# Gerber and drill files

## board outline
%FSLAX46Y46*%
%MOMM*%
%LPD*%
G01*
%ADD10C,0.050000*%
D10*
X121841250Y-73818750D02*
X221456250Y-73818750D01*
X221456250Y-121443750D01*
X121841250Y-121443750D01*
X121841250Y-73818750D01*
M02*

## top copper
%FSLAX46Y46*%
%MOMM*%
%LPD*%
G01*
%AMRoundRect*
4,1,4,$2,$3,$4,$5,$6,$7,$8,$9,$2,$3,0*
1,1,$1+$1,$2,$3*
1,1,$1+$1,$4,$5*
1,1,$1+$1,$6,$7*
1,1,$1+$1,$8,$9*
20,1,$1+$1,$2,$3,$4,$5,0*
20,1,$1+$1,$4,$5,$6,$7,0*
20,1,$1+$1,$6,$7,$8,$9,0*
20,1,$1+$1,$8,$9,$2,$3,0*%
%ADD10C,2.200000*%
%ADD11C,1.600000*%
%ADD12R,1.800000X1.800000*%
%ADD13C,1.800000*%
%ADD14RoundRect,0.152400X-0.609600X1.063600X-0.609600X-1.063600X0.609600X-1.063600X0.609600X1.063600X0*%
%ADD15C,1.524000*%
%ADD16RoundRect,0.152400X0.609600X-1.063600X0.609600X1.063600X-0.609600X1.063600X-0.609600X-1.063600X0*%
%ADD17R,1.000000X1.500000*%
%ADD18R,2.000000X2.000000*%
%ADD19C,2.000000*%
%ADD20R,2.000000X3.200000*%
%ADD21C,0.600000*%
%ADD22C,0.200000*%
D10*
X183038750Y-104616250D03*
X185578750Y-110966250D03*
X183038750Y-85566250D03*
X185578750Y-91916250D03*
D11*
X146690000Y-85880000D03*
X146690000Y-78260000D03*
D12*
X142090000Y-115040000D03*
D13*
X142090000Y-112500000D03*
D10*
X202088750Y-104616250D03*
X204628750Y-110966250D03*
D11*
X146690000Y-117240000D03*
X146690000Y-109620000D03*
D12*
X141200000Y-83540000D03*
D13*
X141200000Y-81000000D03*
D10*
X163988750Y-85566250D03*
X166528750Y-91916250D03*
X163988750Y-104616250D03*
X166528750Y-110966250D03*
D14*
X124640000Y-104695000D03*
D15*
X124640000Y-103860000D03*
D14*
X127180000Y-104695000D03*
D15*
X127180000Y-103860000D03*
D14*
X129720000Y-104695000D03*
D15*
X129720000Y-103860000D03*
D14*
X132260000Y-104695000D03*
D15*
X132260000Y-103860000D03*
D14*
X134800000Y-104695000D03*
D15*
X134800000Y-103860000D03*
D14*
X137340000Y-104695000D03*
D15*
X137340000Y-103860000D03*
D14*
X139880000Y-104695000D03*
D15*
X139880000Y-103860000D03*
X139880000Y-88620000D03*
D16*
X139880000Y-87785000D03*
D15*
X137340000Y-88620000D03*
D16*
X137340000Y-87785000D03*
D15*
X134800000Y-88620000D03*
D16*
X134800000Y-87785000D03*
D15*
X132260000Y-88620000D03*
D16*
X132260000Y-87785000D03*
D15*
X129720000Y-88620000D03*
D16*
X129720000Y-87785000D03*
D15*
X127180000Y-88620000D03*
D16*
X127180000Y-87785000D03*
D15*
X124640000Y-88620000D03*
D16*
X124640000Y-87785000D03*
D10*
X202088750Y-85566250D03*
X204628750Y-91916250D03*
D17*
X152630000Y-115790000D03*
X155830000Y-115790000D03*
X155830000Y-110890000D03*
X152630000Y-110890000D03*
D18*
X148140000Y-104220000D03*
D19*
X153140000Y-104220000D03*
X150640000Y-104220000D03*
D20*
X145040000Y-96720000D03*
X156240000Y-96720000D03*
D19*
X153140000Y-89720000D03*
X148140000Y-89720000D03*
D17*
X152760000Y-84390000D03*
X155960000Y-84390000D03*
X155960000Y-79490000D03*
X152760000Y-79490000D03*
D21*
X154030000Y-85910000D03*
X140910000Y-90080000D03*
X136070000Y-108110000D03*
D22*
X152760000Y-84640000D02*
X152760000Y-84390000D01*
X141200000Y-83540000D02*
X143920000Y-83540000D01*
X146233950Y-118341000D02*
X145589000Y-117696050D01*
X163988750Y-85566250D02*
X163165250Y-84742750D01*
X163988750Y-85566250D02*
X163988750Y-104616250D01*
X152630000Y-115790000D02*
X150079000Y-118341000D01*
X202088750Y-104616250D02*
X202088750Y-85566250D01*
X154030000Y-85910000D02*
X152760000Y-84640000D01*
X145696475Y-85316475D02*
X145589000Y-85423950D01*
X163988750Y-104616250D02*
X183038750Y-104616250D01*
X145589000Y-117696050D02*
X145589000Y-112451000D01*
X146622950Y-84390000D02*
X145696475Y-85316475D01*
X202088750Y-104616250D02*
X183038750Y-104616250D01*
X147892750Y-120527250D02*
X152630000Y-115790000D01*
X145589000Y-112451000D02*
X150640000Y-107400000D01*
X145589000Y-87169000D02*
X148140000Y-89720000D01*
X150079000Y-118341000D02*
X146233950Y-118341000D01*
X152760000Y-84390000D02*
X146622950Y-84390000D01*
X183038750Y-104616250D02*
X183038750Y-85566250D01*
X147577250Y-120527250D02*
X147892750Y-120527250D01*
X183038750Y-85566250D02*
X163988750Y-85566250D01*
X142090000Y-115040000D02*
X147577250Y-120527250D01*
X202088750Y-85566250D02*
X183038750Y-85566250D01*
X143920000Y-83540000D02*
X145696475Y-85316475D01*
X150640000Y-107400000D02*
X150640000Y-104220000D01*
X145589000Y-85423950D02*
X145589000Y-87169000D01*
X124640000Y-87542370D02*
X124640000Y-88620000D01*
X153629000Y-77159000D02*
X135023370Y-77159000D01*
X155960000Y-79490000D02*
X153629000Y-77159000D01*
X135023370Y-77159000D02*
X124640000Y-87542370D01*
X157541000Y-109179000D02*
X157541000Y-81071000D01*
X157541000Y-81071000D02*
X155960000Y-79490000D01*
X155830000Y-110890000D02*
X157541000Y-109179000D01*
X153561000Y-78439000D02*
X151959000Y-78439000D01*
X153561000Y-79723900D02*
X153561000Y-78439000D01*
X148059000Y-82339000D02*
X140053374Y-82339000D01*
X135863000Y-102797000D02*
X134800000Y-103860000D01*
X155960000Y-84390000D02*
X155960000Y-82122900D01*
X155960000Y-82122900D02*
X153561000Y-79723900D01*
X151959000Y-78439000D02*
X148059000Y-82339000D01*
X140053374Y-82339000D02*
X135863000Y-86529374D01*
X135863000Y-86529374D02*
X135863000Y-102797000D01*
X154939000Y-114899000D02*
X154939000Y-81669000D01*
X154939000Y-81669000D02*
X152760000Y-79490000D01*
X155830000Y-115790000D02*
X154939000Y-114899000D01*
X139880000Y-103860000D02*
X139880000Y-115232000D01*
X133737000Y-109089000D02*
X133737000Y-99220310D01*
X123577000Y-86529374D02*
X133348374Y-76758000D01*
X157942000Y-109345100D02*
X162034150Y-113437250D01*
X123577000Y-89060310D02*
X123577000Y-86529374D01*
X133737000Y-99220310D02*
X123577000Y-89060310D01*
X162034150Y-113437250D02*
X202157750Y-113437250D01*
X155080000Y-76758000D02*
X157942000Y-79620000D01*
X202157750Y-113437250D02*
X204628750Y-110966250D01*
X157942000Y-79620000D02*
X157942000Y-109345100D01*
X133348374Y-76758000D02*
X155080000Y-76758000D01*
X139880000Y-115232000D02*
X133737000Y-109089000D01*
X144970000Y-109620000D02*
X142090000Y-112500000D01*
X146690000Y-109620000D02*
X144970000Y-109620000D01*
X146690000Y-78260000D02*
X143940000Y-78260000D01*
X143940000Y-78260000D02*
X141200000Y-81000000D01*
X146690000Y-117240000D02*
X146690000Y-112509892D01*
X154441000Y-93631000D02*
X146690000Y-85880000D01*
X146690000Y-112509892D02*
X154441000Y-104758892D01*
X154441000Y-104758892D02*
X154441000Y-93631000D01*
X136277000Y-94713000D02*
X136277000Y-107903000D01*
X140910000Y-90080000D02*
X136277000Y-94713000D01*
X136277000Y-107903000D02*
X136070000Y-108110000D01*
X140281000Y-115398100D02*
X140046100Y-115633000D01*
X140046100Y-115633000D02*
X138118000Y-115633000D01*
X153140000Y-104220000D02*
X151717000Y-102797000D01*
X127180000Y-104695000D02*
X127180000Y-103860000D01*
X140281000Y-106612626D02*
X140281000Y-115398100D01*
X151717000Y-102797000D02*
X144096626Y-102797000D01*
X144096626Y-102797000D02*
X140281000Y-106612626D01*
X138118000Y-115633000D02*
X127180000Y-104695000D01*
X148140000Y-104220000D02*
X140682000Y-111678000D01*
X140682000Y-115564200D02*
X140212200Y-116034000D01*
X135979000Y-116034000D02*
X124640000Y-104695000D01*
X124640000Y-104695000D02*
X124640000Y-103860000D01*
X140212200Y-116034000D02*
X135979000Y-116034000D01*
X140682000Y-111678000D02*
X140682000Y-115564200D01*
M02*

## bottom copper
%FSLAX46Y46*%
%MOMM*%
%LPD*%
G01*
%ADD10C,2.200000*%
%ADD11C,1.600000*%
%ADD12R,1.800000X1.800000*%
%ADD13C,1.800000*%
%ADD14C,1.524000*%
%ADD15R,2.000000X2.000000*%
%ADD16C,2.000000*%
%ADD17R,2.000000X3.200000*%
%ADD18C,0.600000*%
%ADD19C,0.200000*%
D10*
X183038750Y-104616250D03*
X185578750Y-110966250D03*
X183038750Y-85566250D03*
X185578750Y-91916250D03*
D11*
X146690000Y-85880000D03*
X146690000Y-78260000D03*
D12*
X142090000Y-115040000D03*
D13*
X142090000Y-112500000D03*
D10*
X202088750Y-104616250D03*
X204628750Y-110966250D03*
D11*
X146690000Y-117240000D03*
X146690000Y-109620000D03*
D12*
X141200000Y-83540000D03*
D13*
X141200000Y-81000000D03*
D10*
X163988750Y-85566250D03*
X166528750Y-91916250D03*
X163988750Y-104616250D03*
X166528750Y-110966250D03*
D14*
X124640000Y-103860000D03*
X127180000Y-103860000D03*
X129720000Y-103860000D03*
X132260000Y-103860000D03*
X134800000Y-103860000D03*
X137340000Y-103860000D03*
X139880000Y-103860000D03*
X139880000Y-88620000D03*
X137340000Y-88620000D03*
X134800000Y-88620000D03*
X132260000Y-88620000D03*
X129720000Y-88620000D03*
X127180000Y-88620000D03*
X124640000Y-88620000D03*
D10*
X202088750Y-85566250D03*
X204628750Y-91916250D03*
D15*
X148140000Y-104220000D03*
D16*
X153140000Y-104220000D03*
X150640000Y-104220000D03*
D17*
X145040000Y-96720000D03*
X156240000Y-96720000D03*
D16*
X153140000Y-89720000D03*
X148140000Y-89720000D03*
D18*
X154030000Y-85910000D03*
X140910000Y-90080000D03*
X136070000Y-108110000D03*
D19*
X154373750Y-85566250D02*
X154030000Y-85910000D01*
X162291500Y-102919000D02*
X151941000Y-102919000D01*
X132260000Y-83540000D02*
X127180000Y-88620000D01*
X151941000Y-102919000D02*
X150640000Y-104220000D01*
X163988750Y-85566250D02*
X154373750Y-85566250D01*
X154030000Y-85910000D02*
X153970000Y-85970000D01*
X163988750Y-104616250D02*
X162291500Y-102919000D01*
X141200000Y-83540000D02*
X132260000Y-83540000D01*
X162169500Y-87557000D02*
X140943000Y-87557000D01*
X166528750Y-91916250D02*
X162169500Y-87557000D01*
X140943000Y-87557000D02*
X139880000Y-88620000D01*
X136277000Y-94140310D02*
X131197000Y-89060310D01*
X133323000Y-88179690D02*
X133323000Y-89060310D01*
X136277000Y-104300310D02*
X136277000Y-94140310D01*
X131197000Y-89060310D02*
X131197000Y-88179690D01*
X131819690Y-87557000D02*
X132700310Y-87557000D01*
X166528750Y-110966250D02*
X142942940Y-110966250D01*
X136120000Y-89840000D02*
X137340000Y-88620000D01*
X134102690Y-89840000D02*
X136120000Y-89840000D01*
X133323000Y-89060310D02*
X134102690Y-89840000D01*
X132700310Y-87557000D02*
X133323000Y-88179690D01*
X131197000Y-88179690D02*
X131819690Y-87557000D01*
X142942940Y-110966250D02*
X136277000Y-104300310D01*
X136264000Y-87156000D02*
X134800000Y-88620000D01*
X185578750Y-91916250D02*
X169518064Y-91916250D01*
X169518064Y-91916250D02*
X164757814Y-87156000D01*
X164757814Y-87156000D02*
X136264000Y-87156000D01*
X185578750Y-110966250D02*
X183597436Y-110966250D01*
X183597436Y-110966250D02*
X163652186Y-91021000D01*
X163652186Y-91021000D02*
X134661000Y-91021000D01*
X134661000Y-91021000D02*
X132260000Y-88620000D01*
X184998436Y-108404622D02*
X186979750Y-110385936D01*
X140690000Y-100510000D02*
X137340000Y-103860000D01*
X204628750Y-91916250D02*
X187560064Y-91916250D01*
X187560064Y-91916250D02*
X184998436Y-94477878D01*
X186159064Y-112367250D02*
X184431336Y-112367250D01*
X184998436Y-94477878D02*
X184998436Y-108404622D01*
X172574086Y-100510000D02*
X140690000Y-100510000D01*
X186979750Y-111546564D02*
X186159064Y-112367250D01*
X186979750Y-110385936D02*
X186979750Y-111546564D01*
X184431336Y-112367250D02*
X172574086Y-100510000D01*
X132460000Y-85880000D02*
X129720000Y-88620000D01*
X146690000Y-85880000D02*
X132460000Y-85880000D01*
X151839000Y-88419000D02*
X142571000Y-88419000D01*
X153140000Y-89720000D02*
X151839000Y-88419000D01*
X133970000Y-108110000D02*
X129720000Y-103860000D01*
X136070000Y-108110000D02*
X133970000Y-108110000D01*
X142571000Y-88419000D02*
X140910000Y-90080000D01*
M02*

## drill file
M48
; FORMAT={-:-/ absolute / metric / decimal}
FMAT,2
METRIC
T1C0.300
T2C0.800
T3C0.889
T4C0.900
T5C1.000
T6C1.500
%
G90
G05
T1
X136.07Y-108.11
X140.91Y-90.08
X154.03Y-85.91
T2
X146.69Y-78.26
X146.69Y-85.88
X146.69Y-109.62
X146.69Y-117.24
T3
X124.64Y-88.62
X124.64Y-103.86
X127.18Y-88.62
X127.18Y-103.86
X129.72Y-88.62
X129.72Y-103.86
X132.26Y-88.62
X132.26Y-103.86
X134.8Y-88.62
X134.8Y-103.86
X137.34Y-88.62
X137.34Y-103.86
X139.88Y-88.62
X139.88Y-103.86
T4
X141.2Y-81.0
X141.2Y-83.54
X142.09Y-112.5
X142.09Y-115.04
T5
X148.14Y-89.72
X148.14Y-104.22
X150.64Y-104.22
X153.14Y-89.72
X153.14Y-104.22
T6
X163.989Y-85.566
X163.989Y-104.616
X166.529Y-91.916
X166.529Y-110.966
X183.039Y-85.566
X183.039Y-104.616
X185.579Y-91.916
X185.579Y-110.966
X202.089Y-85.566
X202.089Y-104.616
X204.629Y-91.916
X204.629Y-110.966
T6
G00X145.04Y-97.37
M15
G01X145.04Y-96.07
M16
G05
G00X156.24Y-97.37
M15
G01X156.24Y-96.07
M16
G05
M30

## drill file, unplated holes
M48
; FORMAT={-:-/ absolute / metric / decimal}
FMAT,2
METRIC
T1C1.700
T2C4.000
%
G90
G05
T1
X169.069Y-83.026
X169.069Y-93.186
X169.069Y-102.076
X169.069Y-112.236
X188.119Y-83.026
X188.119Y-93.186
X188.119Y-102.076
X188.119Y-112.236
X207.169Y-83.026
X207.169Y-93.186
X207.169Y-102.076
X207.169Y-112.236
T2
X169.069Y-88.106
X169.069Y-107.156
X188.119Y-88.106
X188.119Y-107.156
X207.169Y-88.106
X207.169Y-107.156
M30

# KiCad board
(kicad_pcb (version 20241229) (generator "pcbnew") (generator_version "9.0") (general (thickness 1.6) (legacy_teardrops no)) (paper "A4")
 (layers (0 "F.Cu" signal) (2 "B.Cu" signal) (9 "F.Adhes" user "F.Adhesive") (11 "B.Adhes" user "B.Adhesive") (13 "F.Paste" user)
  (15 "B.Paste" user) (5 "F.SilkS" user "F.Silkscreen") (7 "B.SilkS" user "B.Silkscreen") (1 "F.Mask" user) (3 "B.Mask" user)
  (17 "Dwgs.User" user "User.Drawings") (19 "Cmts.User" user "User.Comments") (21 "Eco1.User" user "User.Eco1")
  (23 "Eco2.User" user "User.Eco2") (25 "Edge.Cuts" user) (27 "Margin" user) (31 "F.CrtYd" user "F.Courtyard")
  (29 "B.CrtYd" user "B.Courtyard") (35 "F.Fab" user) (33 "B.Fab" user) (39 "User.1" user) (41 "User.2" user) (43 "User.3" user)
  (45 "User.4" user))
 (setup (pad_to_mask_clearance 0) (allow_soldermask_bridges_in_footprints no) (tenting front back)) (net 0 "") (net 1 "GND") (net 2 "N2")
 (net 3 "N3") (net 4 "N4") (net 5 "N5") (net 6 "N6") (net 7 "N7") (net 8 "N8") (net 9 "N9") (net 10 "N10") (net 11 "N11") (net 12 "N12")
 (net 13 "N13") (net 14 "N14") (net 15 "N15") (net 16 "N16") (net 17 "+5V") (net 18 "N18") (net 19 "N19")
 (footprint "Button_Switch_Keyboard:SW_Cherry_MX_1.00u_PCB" (layer "F.Cu") (at 183.03875 104.61625 90)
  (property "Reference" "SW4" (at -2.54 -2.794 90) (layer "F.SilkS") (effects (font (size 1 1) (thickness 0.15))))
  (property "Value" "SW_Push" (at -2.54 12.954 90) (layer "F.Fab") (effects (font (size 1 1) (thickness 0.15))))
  (pad "" np_thru_hole circle (at -7.62 5.08 90) (size 1.7 1.7) (drill 1.7) (layers "*.Cu" "*.Mask"))
  (pad "" np_thru_hole circle (at -2.54 5.08 90) (size 4 4) (drill 4) (layers "*.Cu" "*.Mask"))
  (pad "" np_thru_hole circle (at 2.54 5.08 90) (size 1.7 1.7) (drill 1.7) (layers "*.Cu" "*.Mask"))
  (pad "1" thru_hole circle (at 0 0 90) (size 2.2 2.2) (drill 1.5) (layers "*.Cu" "*.Mask") (remove_unused_layers no) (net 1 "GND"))
  (pad "2" thru_hole circle (at -6.35 2.54 90) (size 2.2 2.2) (drill 1.5) (layers "*.Cu" "*.Mask") (remove_unused_layers no) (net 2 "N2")))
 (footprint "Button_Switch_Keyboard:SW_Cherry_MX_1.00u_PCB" (layer "F.Cu") (at 183.03875 85.56625 90)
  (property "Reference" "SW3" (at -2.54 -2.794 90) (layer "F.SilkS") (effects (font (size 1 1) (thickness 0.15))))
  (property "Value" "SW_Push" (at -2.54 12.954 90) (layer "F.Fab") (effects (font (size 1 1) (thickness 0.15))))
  (pad "" np_thru_hole circle (at -7.62 5.08 90) (size 1.7 1.7) (drill 1.7) (layers "*.Cu" "*.Mask"))
  (pad "" np_thru_hole circle (at -2.54 5.08 90) (size 4 4) (drill 4) (layers "*.Cu" "*.Mask"))
  (pad "" np_thru_hole circle (at 2.54 5.08 90) (size 1.7 1.7) (drill 1.7) (layers "*.Cu" "*.Mask"))
  (pad "1" thru_hole circle (at 0 0 90) (size 2.2 2.2) (drill 1.5) (layers "*.Cu" "*.Mask") (remove_unused_layers no) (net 1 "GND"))
  (pad "2" thru_hole circle (at -6.35 2.54 90) (size 2.2 2.2) (drill 1.5) (layers "*.Cu" "*.Mask") (remove_unused_layers no) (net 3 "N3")))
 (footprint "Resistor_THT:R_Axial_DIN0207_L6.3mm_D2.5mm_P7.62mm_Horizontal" (layer "F.Cu") (at 146.69 85.88 90)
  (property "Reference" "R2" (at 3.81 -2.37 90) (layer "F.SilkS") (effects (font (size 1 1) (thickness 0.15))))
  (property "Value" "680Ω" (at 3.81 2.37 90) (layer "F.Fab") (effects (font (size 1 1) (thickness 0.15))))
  (pad "1" thru_hole circle (at 0 0 90) (size 1.6 1.6) (drill 0.8) (layers "*.Cu" "*.Mask") (remove_unused_layers no) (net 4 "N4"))
  (pad "2" thru_hole circle (at 7.62 0 90) (size 1.6 1.6) (drill 0.8) (layers "*.Cu" "*.Mask") (remove_unused_layers no) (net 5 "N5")))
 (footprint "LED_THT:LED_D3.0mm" (layer "F.Cu") (at 142.09 115.04 90)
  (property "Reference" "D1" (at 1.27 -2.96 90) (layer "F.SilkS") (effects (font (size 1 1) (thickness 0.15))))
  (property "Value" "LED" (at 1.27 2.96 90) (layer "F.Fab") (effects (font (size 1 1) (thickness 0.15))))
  (pad "1" thru_hole rect (at 0 0 90) (size 1.8 1.8) (drill 0.9) (layers "*.Cu" "*.Mask") (remove_unused_layers no) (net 1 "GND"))
  (pad "2" thru_hole circle (at 2.54 0 90) (size 1.8 1.8) (drill 0.9) (layers "*.Cu" "*.Mask") (remove_unused_layers no) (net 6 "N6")))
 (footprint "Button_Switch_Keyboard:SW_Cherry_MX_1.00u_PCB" (layer "F.Cu") (at 202.08875 104.61625 90)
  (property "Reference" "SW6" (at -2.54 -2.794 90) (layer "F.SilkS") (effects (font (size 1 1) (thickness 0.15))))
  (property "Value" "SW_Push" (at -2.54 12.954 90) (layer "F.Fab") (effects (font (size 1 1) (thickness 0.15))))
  (pad "" np_thru_hole circle (at -7.62 5.08 90) (size 1.7 1.7) (drill 1.7) (layers "*.Cu" "*.Mask"))
  (pad "" np_thru_hole circle (at -2.54 5.08 90) (size 4 4) (drill 4) (layers "*.Cu" "*.Mask"))
  (pad "" np_thru_hole circle (at 2.54 5.08 90) (size 1.7 1.7) (drill 1.7) (layers "*.Cu" "*.Mask"))
  (pad "1" thru_hole circle (at 0 0 90) (size 2.2 2.2) (drill 1.5) (layers "*.Cu" "*.Mask") (remove_unused_layers no) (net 1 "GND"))
  (pad "2" thru_hole circle (at -6.35 2.54 90) (size 2.2 2.2) (drill 1.5) (layers "*.Cu" "*.Mask") (remove_unused_layers no) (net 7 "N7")))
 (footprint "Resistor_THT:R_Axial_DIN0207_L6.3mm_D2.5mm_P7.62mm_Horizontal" (layer "F.Cu") (at 146.69 117.24 90)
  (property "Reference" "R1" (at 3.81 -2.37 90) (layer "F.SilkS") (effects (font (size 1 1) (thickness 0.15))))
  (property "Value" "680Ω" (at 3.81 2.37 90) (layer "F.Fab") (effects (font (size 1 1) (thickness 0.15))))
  (pad "1" thru_hole circle (at 0 0 90) (size 1.6 1.6) (drill 0.8) (layers "*.Cu" "*.Mask") (remove_unused_layers no) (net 4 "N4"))
  (pad "2" thru_hole circle (at 7.62 0 90) (size 1.6 1.6) (drill 0.8) (layers "*.Cu" "*.Mask") (remove_unused_layers no) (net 6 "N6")))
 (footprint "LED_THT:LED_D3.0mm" (layer "F.Cu") (at 141.2 83.54 90)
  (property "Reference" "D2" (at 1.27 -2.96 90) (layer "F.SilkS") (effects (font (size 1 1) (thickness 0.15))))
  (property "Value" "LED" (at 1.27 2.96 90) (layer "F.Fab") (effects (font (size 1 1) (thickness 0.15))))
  (pad "1" thru_hole rect (at 0 0 90) (size 1.8 1.8) (drill 0.9) (layers "*.Cu" "*.Mask") (remove_unused_layers no) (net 1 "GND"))
  (pad "2" thru_hole circle (at 2.54 0 90) (size 1.8 1.8) (drill 0.9) (layers "*.Cu" "*.Mask") (remove_unused_layers no) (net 5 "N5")))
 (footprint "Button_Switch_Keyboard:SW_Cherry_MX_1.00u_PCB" (layer "F.Cu") (at 163.98875 85.56625 90)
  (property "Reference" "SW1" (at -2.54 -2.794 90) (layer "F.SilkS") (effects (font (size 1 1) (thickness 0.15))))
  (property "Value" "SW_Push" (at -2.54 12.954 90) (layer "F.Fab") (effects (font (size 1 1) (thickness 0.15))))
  (pad "" np_thru_hole circle (at -7.62 5.08 90) (size 1.7 1.7) (drill 1.7) (layers "*.Cu" "*.Mask"))
  (pad "" np_thru_hole circle (at -2.54 5.08 90) (size 4 4) (drill 4) (layers "*.Cu" "*.Mask"))
  (pad "" np_thru_hole circle (at 2.54 5.08 90) (size 1.7 1.7) (drill 1.7) (layers "*.Cu" "*.Mask"))
  (pad "1" thru_hole circle (at 0 0 90) (size 2.2 2.2) (drill 1.5) (layers "*.Cu" "*.Mask") (remove_unused_layers no) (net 1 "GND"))
  (pad "2" thru_hole circle (at -6.35 2.54 90) (size 2.2 2.2) (drill 1.5) (layers "*.Cu" "*.Mask") (remove_unused_layers no) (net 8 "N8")))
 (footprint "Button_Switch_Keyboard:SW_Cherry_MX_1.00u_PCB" (layer "F.Cu") (at 163.98875 104.61625 90)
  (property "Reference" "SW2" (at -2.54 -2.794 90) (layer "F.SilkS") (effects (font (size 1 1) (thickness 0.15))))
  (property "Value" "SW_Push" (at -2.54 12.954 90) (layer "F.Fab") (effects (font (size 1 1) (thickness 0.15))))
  (pad "" np_thru_hole circle (at -7.62 5.08 90) (size 1.7 1.7) (drill 1.7) (layers "*.Cu" "*.Mask"))
  (pad "" np_thru_hole circle (at -2.54 5.08 90) (size 4 4) (drill 4) (layers "*.Cu" "*.Mask"))
  (pad "" np_thru_hole circle (at 2.54 5.08 90) (size 1.7 1.7) (drill 1.7) (layers "*.Cu" "*.Mask"))
  (pad "1" thru_hole circle (at 0 0 90) (size 2.2 2.2) (drill 1.5) (layers "*.Cu" "*.Mask") (remove_unused_layers no) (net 1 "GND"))
  (pad "2" thru_hole circle (at -6.35 2.54 90) (size 2.2 2.2) (drill 1.5) (layers "*.Cu" "*.Mask") (remove_unused_layers no) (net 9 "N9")))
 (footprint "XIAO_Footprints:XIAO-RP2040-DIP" (layer "F.Cu") (at 132.26 96.24 90)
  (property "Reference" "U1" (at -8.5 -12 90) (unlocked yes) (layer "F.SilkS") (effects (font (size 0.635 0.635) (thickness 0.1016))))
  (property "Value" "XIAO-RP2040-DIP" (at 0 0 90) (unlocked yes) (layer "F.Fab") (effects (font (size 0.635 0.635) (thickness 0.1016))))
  (pad "1" smd roundrect (at -8.455 -7.62 270) (size 2.432 1.524) (layers "F.Cu" "F.Mask") (roundrect_rratio 0.1) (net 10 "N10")
   (thermal_bridge_angle 45))
  (pad "1" thru_hole circle (at -7.62 -7.62 270) (size 1.524 1.524) (drill 0.889) (layers "*.Cu" "*.Mask") (remove_unused_layers no)
   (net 10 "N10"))
  (pad "2" smd roundrect (at -8.455 -5.08 270) (size 2.432 1.524) (layers "F.Cu" "F.Mask") (roundrect_rratio 0.1) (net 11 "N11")
   (thermal_bridge_angle 45))
  (pad "2" thru_hole circle (at -7.62 -5.08 270) (size 1.524 1.524) (drill 0.889) (layers "*.Cu" "*.Mask") (remove_unused_layers no)
   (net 11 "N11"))
  (pad "3" smd roundrect (at -8.455 -2.54 270) (size 2.432 1.524) (layers "F.Cu" "F.Mask") (roundrect_rratio 0.1) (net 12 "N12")
   (thermal_bridge_angle 45))
  (pad "3" thru_hole circle (at -7.62 -2.54 270) (size 1.524 1.524) (drill 0.889) (layers "*.Cu" "*.Mask") (remove_unused_layers no)
   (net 12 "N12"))
  (pad "4" smd roundrect (at -8.455 0 270) (size 2.432 1.524) (layers "F.Cu" "F.Mask") (roundrect_rratio 0.1) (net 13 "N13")
   (thermal_bridge_angle 45))
  (pad "4" thru_hole circle (at -7.62 0 270) (size 1.524 1.524) (drill 0.889) (layers "*.Cu" "*.Mask") (remove_unused_layers no)
   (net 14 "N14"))
  (pad "5" smd roundrect (at -8.455 2.54 270) (size 2.432 1.524) (layers "F.Cu" "F.Mask") (roundrect_rratio 0.1) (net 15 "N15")
   (thermal_bridge_angle 45))
  (pad "5" thru_hole circle (at -7.62 2.54 270) (size 1.524 1.524) (drill 0.889) (layers "*.Cu" "*.Mask") (remove_unused_layers no)
   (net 15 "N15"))
  (pad "6" smd roundrect (at -8.455 5.08 270) (size 2.432 1.524) (layers "F.Cu" "F.Mask") (roundrect_rratio 0.1) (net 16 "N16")
   (thermal_bridge_angle 45))
  (pad "6" thru_hole circle (at -7.62 5.08 270) (size 1.524 1.524) (drill 0.889) (layers "*.Cu" "*.Mask") (remove_unused_layers no)
   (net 16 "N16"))
  (pad "7" smd roundrect (at -8.455 7.62 270) (size 2.432 1.524) (layers "F.Cu" "F.Mask") (roundrect_rratio 0.1) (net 7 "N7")
   (thermal_bridge_angle 45))
  (pad "7" thru_hole circle (at -7.62 7.62 270) (size 1.524 1.524) (drill 0.889) (layers "*.Cu" "*.Mask") (remove_unused_layers no)
   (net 7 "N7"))
  (pad "8" thru_hole circle (at 7.62 7.62 90) (size 1.524 1.524) (drill 0.889) (layers "*.Cu" "*.Mask") (remove_unused_layers no)
   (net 8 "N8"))
  (pad "8" smd roundrect (at 8.455 7.62 90) (size 2.432 1.524) (layers "F.Cu" "F.Mask") (roundrect_rratio 0.1) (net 8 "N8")
   (thermal_bridge_angle 45))
  (pad "9" thru_hole circle (at 7.62 5.08 90) (size 1.524 1.524) (drill 0.889) (layers "*.Cu" "*.Mask") (remove_unused_layers no)
   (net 9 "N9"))
  (pad "9" smd roundrect (at 8.455 5.08 90) (size 2.432 1.524) (layers "F.Cu" "F.Mask") (roundrect_rratio 0.1) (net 9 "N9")
   (thermal_bridge_angle 45))
  (pad "10" thru_hole circle (at 7.62 2.54 90) (size 1.524 1.524) (drill 0.889) (layers "*.Cu" "*.Mask") (remove_unused_layers no)
   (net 3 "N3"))
  (pad "10" smd roundrect (at 8.455 2.54 90) (size 2.432 1.524) (layers "F.Cu" "F.Mask") (roundrect_rratio 0.1) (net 3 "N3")
   (thermal_bridge_angle 45))
  (pad "11" thru_hole circle (at 7.62 0 90) (size 1.524 1.524) (drill 0.889) (layers "*.Cu" "*.Mask") (remove_unused_layers no) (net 2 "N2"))
  (pad "11" smd roundrect (at 8.455 0 90) (size 2.432 1.524) (layers "F.Cu" "F.Mask") (roundrect_rratio 0.1) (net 2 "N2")
   (thermal_bridge_angle 45))
  (pad "12" thru_hole circle (at 7.62 -2.54 90) (size 1.524 1.524) (drill 0.889) (layers "*.Cu" "*.Mask") (remove_unused_layers no)
   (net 4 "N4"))
  (pad "12" smd roundrect (at 8.455 -2.54 90) (size 2.432 1.524) (layers "F.Cu" "F.Mask") (roundrect_rratio 0.1) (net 4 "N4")
   (thermal_bridge_angle 45))
  (pad "13" thru_hole circle (at 7.62 -5.08 90) (size 1.524 1.524) (drill 0.889) (layers "*.Cu" "*.Mask") (remove_unused_layers no)
   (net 1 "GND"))
  (pad "13" smd roundrect (at 8.455 -5.08 90) (size 2.432 1.524) (layers "F.Cu" "F.Mask") (roundrect_rratio 0.1) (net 1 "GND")
   (thermal_bridge_angle 45))
  (pad "14" thru_hole circle (at 7.62 -7.62 90) (size 1.524 1.524) (drill 0.889) (layers "*.Cu" "*.Mask") (remove_unused_layers no)
   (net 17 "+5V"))
  (pad "14" smd roundrect (at 8.455 -7.62 90) (size 2.432 1.524) (layers "F.Cu" "F.Mask") (roundrect_rratio 0.1) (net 17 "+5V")
   (thermal_bridge_angle 45)))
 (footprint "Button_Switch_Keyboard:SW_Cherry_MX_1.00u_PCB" (layer "F.Cu") (at 202.08875 85.56625 90)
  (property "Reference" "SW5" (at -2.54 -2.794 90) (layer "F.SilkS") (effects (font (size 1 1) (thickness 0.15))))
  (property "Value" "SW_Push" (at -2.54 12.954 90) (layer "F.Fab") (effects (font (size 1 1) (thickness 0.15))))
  (pad "" np_thru_hole circle (at -7.62 5.08 90) (size 1.7 1.7) (drill 1.7) (layers "*.Cu" "*.Mask"))
  (pad "" np_thru_hole circle (at -2.54 5.08 90) (size 4 4) (drill 4) (layers "*.Cu" "*.Mask"))
  (pad "" np_thru_hole circle (at 2.54 5.08 90) (size 1.7 1.7) (drill 1.7) (layers "*.Cu" "*.Mask"))
  (pad "1" thru_hole circle (at 0 0 90) (size 2.2 2.2) (drill 1.5) (layers "*.Cu" "*.Mask") (remove_unused_layers no) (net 1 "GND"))
  (pad "2" thru_hole circle (at -6.35 2.54 90) (size 2.2 2.2) (drill 1.5) (layers "*.Cu" "*.Mask") (remove_unused_layers no) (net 16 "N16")))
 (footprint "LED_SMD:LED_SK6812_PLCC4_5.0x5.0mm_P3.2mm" (layer "F.Cu") (at 154.23 113.34 90)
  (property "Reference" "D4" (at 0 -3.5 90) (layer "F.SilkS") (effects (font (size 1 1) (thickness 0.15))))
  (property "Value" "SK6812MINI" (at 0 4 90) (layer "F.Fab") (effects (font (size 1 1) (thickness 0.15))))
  (pad "1" smd rect (at -2.45 -1.6 270) (size 1.5 1) (layers "F.Cu" "F.Mask" "F.Paste") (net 1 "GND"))
  (pad "2" smd rect (at -2.45 1.6 270) (size 1.5 1) (layers "F.Cu" "F.Mask" "F.Paste") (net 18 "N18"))
  (pad "3" smd rect (at 2.45 1.6 270) (size 1.5 1) (layers "F.Cu" "F.Mask" "F.Paste") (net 17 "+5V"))
  (pad "4" smd rect (at 2.45 -1.6 270) (size 1.5 1) (layers "F.Cu" "F.Mask" "F.Paste") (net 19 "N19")))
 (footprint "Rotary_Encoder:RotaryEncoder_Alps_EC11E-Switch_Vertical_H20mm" (layer "F.Cu") (at 148.14 104.22 90)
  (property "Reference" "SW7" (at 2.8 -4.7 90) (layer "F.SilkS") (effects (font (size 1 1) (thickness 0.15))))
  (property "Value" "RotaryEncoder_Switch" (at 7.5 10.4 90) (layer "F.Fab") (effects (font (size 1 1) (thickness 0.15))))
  (pad "A" thru_hole rect (at 0 0 90) (size 2 2) (drill 1) (layers "*.Cu" "*.Mask") (remove_unused_layers no) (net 10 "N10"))
  (pad "B" thru_hole circle (at 0 5 90) (size 2 2) (drill 1) (layers "*.Cu" "*.Mask") (remove_unused_layers no) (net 11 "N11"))
  (pad "C" thru_hole circle (at 0 2.5 90) (size 2 2) (drill 1) (layers "*.Cu" "*.Mask") (remove_unused_layers no) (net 1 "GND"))
  (pad "MP" thru_hole rect (at 7.5 -3.1 90) (size 3.2 2) (drill oval 2.8 1.5) (layers "*.Cu" "*.Mask") (remove_unused_layers no))
  (pad "MP" thru_hole rect (at 7.5 8.1 90) (size 3.2 2) (drill oval 2.8 1.5) (layers "*.Cu" "*.Mask") (remove_unused_layers no))
  (pad "S1" thru_hole circle (at 14.5 5 90) (size 2 2) (drill 1) (layers "*.Cu" "*.Mask") (remove_unused_layers no) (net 12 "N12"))
  (pad "S2" thru_hole circle (at 14.5 0 90) (size 2 2) (drill 1) (layers "*.Cu" "*.Mask") (remove_unused_layers no) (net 1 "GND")))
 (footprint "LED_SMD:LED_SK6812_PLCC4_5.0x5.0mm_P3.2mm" (layer "F.Cu") (at 154.36 81.94 90)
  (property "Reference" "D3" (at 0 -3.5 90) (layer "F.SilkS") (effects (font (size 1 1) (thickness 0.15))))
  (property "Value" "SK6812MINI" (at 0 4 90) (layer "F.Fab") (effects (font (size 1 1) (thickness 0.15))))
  (pad "1" smd rect (at -2.45 -1.6 270) (size 1.5 1) (layers "F.Cu" "F.Mask" "F.Paste") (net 1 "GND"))
  (pad "2" smd rect (at -2.45 1.6 270) (size 1.5 1) (layers "F.Cu" "F.Mask" "F.Paste") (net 15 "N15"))
  (pad "3" smd rect (at 2.45 1.6 270) (size 1.5 1) (layers "F.Cu" "F.Mask" "F.Paste") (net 17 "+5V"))
  (pad "4" smd rect (at 2.45 -1.6 270) (size 1.5 1) (layers "F.Cu" "F.Mask" "F.Paste") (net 18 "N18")))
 (gr_rect (start 121.84125 73.81875) (end 221.45625 121.44375) (stroke (width 0.05) (type default)) (fill no) (layer "Edge.Cuts"))
 (segment (start 152.76 84.64) (end 152.76 84.39) (width 0.2) (layer "F.Cu") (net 1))
 (segment (start 141.2 83.54) (end 143.92 83.54) (width 0.2) (layer "F.Cu") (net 1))
 (segment (start 146.23395 118.341) (end 145.589 117.69605) (width 0.2) (layer "F.Cu") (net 1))
 (segment (start 163.98875 85.56625) (end 163.16525 84.74275) (width 0.2) (layer "F.Cu") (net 1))
 (segment (start 163.98875 85.56625) (end 163.98875 104.61625) (width 0.2) (layer "F.Cu") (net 1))
 (segment (start 152.63 115.79) (end 150.079 118.341) (width 0.2) (layer "F.Cu") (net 1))
 (segment (start 202.08875 104.61625) (end 202.08875 85.56625) (width 0.2) (layer "F.Cu") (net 1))
 (segment (start 154.03 85.91) (end 152.76 84.64) (width 0.2) (layer "F.Cu") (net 1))
 (segment (start 145.696475 85.316475) (end 145.589 85.42395) (width 0.2) (layer "F.Cu") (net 1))
 (segment (start 163.98875 104.61625) (end 183.03875 104.61625) (width 0.2) (layer "F.Cu") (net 1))
 (segment (start 145.589 117.69605) (end 145.589 112.451) (width 0.2) (layer "F.Cu") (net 1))
 (segment (start 146.62295 84.39) (end 145.696475 85.316475) (width 0.2) (layer "F.Cu") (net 1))
 (segment (start 202.08875 104.61625) (end 183.03875 104.61625) (width 0.2) (layer "F.Cu") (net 1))
 (segment (start 147.89275 120.52725) (end 152.63 115.79) (width 0.2) (layer "F.Cu") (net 1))
 (segment (start 145.589 112.451) (end 150.64 107.4) (width 0.2) (layer "F.Cu") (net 1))
 (segment (start 145.589 87.169) (end 148.14 89.72) (width 0.2) (layer "F.Cu") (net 1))
 (segment (start 150.079 118.341) (end 146.23395 118.341) (width 0.2) (layer "F.Cu") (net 1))
 (segment (start 152.76 84.39) (end 146.62295 84.39) (width 0.2) (layer "F.Cu") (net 1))
 (segment (start 183.03875 104.61625) (end 183.03875 85.56625) (width 0.2) (layer "F.Cu") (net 1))
 (segment (start 147.57725 120.52725) (end 147.89275 120.52725) (width 0.2) (layer "F.Cu") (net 1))
 (segment (start 183.03875 85.56625) (end 163.98875 85.56625) (width 0.2) (layer "F.Cu") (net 1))
 (segment (start 142.09 115.04) (end 147.57725 120.52725) (width 0.2) (layer "F.Cu") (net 1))
 (segment (start 202.08875 85.56625) (end 183.03875 85.56625) (width 0.2) (layer "F.Cu") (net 1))
 (segment (start 143.92 83.54) (end 145.696475 85.316475) (width 0.2) (layer "F.Cu") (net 1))
 (segment (start 150.64 107.4) (end 150.64 104.22) (width 0.2) (layer "F.Cu") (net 1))
 (segment (start 145.589 85.42395) (end 145.589 87.169) (width 0.2) (layer "F.Cu") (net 1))
 (via (at 154.03 85.91) (size 0.6) (drill 0.3) (layers "F.Cu" "B.Cu") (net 1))
 (segment (start 154.37375 85.56625) (end 154.03 85.91) (width 0.2) (layer "B.Cu") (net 1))
 (segment (start 162.2915 102.919) (end 151.941 102.919) (width 0.2) (layer "B.Cu") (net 1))
 (segment (start 132.26 83.54) (end 127.18 88.62) (width 0.2) (layer "B.Cu") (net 1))
 (segment (start 151.941 102.919) (end 150.64 104.22) (width 0.2) (layer "B.Cu") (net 1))
 (segment (start 163.98875 85.56625) (end 154.37375 85.56625) (width 0.2) (layer "B.Cu") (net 1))
 (segment (start 154.03 85.91) (end 153.97 85.97) (width 0.2) (layer "B.Cu") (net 1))
 (segment (start 163.98875 104.61625) (end 162.2915 102.919) (width 0.2) (layer "B.Cu") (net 1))
 (segment (start 141.2 83.54) (end 132.26 83.54) (width 0.2) (layer "B.Cu") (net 1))
 (segment (start 124.64 87.54237) (end 124.64 88.62) (width 0.2) (layer "F.Cu") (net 17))
 (segment (start 153.629 77.159) (end 135.02337 77.159) (width 0.2) (layer "F.Cu") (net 17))
 (segment (start 155.96 79.49) (end 153.629 77.159) (width 0.2) (layer "F.Cu") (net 17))
 (segment (start 135.02337 77.159) (end 124.64 87.54237) (width 0.2) (layer "F.Cu") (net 17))
 (segment (start 157.541 109.179) (end 157.541 81.071) (width 0.2) (layer "F.Cu") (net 17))
 (segment (start 157.541 81.071) (end 155.96 79.49) (width 0.2) (layer "F.Cu") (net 17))
 (segment (start 155.83 110.89) (end 157.541 109.179) (width 0.2) (layer "F.Cu") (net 17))
 (segment (start 153.561 78.439) (end 151.959 78.439) (width 0.2) (layer "F.Cu") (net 15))
 (segment (start 153.561 79.7239) (end 153.561 78.439) (width 0.2) (layer "F.Cu") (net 15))
 (segment (start 148.059 82.339) (end 140.053374 82.339) (width 0.2) (layer "F.Cu") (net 15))
 (segment (start 135.863 102.797) (end 134.8 103.86) (width 0.2) (layer "F.Cu") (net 15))
 (segment (start 155.96 84.39) (end 155.96 82.1229) (width 0.2) (layer "F.Cu") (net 15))
 (segment (start 155.96 82.1229) (end 153.561 79.7239) (width 0.2) (layer "F.Cu") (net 15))
 (segment (start 151.959 78.439) (end 148.059 82.339) (width 0.2) (layer "F.Cu") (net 15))
 (segment (start 140.053374 82.339) (end 135.863 86.529374) (width 0.2) (layer "F.Cu") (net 15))
 (segment (start 135.863 86.529374) (end 135.863 102.797) (width 0.2) (layer "F.Cu") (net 15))
 (segment (start 154.939 114.899) (end 154.939 81.669) (width 0.2) (layer "F.Cu") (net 18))
 (segment (start 154.939 81.669) (end 152.76 79.49) (width 0.2) (layer "F.Cu") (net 18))
 (segment (start 155.83 115.79) (end 154.939 114.899) (width 0.2) (layer "F.Cu") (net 18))
 (segment (start 162.1695 87.557) (end 140.943 87.557) (width 0.2) (layer "B.Cu") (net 8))
 (segment (start 166.52875 91.91625) (end 162.1695 87.557) (width 0.2) (layer "B.Cu") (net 8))
 (segment (start 140.943 87.557) (end 139.88 88.62) (width 0.2) (layer "B.Cu") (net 8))
 (segment (start 136.277 94.14031) (end 131.197 89.06031) (width 0.2) (layer "B.Cu") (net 9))
 (segment (start 133.323 88.17969) (end 133.323 89.06031) (width 0.2) (layer "B.Cu") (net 9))
 (segment (start 136.277 104.30031) (end 136.277 94.14031) (width 0.2) (layer "B.Cu") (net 9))
 (segment (start 131.197 89.06031) (end 131.197 88.17969) (width 0.2) (layer "B.Cu") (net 9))
 (segment (start 131.81969 87.557) (end 132.70031 87.557) (width 0.2) (layer "B.Cu") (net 9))
 (segment (start 166.52875 110.96625) (end 142.94294 110.96625) (width 0.2) (layer "B.Cu") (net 9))
 (segment (start 136.12 89.84) (end 137.34 88.62) (width 0.2) (layer "B.Cu") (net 9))
 (segment (start 134.10269 89.84) (end 136.12 89.84) (width 0.2) (layer "B.Cu") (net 9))
 (segment (start 133.323 89.06031) (end 134.10269 89.84) (width 0.2) (layer "B.Cu") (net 9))
 (segment (start 132.70031 87.557) (end 133.323 88.17969) (width 0.2) (layer "B.Cu") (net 9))
 (segment (start 131.197 88.17969) (end 131.81969 87.557) (width 0.2) (layer "B.Cu") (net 9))
 (segment (start 142.94294 110.96625) (end 136.277 104.30031) (width 0.2) (layer "B.Cu") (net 9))
 (segment (start 136.264 87.156) (end 134.8 88.62) (width 0.2) (layer "B.Cu") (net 3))
 (segment (start 185.57875 91.91625) (end 169.518064 91.91625) (width 0.2) (layer "B.Cu") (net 3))
 (segment (start 169.518064 91.91625) (end 164.757814 87.156) (width 0.2) (layer "B.Cu") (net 3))
 (segment (start 164.757814 87.156) (end 136.264 87.156) (width 0.2) (layer "B.Cu") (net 3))
 (segment (start 185.57875 110.96625) (end 183.597436 110.96625) (width 0.2) (layer "B.Cu") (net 2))
 (segment (start 183.597436 110.96625) (end 163.652186 91.021) (width 0.2) (layer "B.Cu") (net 2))
 (segment (start 163.652186 91.021) (end 134.661 91.021) (width 0.2) (layer "B.Cu") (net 2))
 (segment (start 134.661 91.021) (end 132.26 88.62) (width 0.2) (layer "B.Cu") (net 2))
 (segment (start 184.998436 108.404622) (end 186.97975 110.385936) (width 0.2) (layer "B.Cu") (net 16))
 (segment (start 140.69 100.51) (end 137.34 103.86) (width 0.2) (layer "B.Cu") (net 16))
 (segment (start 204.62875 91.91625) (end 187.560064 91.91625) (width 0.2) (layer "B.Cu") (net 16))
 (segment (start 187.560064 91.91625) (end 184.998436 94.477878) (width 0.2) (layer "B.Cu") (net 16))
 (segment (start 186.159064 112.36725) (end 184.431336 112.36725) (width 0.2) (layer "B.Cu") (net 16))
 (segment (start 184.998436 94.477878) (end 184.998436 108.404622) (width 0.2) (layer "B.Cu") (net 16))
 (segment (start 172.574086 100.51) (end 140.69 100.51) (width 0.2) (layer "B.Cu") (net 16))
 (segment (start 186.97975 111.546564) (end 186.159064 112.36725) (width 0.2) (layer "B.Cu") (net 16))
 (segment (start 186.97975 110.385936) (end 186.97975 111.546564) (width 0.2) (layer "B.Cu") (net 16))
 (segment (start 184.431336 112.36725) (end 172.574086 100.51) (width 0.2) (layer "B.Cu") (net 16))
 (segment (start 139.88 103.86) (end 139.88 115.232) (width 0.2) (layer "F.Cu") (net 7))
 (segment (start 133.737 109.089) (end 133.737 99.22031) (width 0.2) (layer "F.Cu") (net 7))
 (segment (start 123.577 86.529374) (end 133.348374 76.758) (width 0.2) (layer "F.Cu") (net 7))
 (segment (start 157.942 109.3451) (end 162.03415 113.43725) (width 0.2) (layer "F.Cu") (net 7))
 (segment (start 123.577 89.06031) (end 123.577 86.529374) (width 0.2) (layer "F.Cu") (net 7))
 (segment (start 133.737 99.22031) (end 123.577 89.06031) (width 0.2) (layer "F.Cu") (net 7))
 (segment (start 162.03415 113.43725) (end 202.15775 113.43725) (width 0.2) (layer "F.Cu") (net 7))
 (segment (start 155.08 76.758) (end 157.942 79.62) (width 0.2) (layer "F.Cu") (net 7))
 (segment (start 202.15775 113.43725) (end 204.62875 110.96625) (width 0.2) (layer "F.Cu") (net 7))
 (segment (start 157.942 79.62) (end 157.942 109.3451) (width 0.2) (layer "F.Cu") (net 7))
 (segment (start 133.348374 76.758) (end 155.08 76.758) (width 0.2) (layer "F.Cu") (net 7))
 (segment (start 139.88 115.232) (end 133.737 109.089) (width 0.2) (layer "F.Cu") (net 7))
 (segment (start 144.97 109.62) (end 142.09 112.5) (width 0.2) (layer "F.Cu") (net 6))
 (segment (start 146.69 109.62) (end 144.97 109.62) (width 0.2) (layer "F.Cu") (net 6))
 (segment (start 146.69 78.26) (end 143.94 78.26) (width 0.2) (layer "F.Cu") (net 5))
 (segment (start 143.94 78.26) (end 141.2 81) (width 0.2) (layer "F.Cu") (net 5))
 (segment (start 146.69 117.24) (end 146.69 112.509892) (width 0.2) (layer "F.Cu") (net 4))
 (segment (start 154.441 93.631) (end 146.69 85.88) (width 0.2) (layer "F.Cu") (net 4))
 (segment (start 146.69 112.509892) (end 154.441 104.758892) (width 0.2) (layer "F.Cu") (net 4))
 (segment (start 154.441 104.758892) (end 154.441 93.631) (width 0.2) (layer "F.Cu") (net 4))
 (segment (start 132.46 85.88) (end 129.72 88.62) (width 0.2) (layer "B.Cu") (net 4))
 (segment (start 146.69 85.88) (end 132.46 85.88) (width 0.2) (layer "B.Cu") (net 4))
 (segment (start 136.277 94.713) (end 136.277 107.903) (width 0.2) (layer "F.Cu") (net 12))
 (segment (start 140.91 90.08) (end 136.277 94.713) (width 0.2) (layer "F.Cu") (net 12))
 (segment (start 136.277 107.903) (end 136.07 108.11) (width 0.2) (layer "F.Cu") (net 12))
 (via (at 140.91 90.08) (size 0.6) (drill 0.3) (layers "F.Cu" "B.Cu") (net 12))
 (via (at 136.07 108.11) (size 0.6) (drill 0.3) (layers "F.Cu" "B.Cu") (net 12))
 (segment (start 151.839 88.419) (end 142.571 88.419) (width 0.2) (layer "B.Cu") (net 12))
 (segment (start 153.14 89.72) (end 151.839 88.419) (width 0.2) (layer "B.Cu") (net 12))
 (segment (start 133.97 108.11) (end 129.72 103.86) (width 0.2) (layer "B.Cu") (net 12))
 (segment (start 136.07 108.11) (end 133.97 108.11) (width 0.2) (layer "B.Cu") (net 12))
 (segment (start 142.571 88.419) (end 140.91 90.08) (width 0.2) (layer "B.Cu") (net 12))
 (segment (start 140.281 115.3981) (end 140.0461 115.633) (width 0.2) (layer "F.Cu") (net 11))
 (segment (start 140.0461 115.633) (end 138.118 115.633) (width 0.2) (layer "F.Cu") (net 11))
 (segment (start 153.14 104.22) (end 151.717 102.797) (width 0.2) (layer "F.Cu") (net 11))
 (segment (start 127.18 104.695) (end 127.18 103.86) (width 0.2) (layer "F.Cu") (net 11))
 (segment (start 140.281 106.612626) (end 140.281 115.3981) (width 0.2) (layer "F.Cu") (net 11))
 (segment (start 151.717 102.797) (end 144.096626 102.797) (width 0.2) (layer "F.Cu") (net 11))
 (segment (start 144.096626 102.797) (end 140.281 106.612626) (width 0.2) (layer "F.Cu") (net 11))
 (segment (start 138.118 115.633) (end 127.18 104.695) (width 0.2) (layer "F.Cu") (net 11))
 (segment (start 148.14 104.22) (end 140.682 111.678) (width 0.2) (layer "F.Cu") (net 10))
 (segment (start 140.682 115.5642) (end 140.2122 116.034) (width 0.2) (layer "F.Cu") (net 10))
 (segment (start 135.979 116.034) (end 124.64 104.695) (width 0.2) (layer "F.Cu") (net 10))
 (segment (start 124.64 104.695) (end 124.64 103.86) (width 0.2) (layer "F.Cu") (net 10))
 (segment (start 140.2122 116.034) (end 135.979 116.034) (width 0.2) (layer "F.Cu") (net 10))
 (segment (start 140.682 111.678) (end 140.682 115.5642) (width 0.2) (layer "F.Cu") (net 10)))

